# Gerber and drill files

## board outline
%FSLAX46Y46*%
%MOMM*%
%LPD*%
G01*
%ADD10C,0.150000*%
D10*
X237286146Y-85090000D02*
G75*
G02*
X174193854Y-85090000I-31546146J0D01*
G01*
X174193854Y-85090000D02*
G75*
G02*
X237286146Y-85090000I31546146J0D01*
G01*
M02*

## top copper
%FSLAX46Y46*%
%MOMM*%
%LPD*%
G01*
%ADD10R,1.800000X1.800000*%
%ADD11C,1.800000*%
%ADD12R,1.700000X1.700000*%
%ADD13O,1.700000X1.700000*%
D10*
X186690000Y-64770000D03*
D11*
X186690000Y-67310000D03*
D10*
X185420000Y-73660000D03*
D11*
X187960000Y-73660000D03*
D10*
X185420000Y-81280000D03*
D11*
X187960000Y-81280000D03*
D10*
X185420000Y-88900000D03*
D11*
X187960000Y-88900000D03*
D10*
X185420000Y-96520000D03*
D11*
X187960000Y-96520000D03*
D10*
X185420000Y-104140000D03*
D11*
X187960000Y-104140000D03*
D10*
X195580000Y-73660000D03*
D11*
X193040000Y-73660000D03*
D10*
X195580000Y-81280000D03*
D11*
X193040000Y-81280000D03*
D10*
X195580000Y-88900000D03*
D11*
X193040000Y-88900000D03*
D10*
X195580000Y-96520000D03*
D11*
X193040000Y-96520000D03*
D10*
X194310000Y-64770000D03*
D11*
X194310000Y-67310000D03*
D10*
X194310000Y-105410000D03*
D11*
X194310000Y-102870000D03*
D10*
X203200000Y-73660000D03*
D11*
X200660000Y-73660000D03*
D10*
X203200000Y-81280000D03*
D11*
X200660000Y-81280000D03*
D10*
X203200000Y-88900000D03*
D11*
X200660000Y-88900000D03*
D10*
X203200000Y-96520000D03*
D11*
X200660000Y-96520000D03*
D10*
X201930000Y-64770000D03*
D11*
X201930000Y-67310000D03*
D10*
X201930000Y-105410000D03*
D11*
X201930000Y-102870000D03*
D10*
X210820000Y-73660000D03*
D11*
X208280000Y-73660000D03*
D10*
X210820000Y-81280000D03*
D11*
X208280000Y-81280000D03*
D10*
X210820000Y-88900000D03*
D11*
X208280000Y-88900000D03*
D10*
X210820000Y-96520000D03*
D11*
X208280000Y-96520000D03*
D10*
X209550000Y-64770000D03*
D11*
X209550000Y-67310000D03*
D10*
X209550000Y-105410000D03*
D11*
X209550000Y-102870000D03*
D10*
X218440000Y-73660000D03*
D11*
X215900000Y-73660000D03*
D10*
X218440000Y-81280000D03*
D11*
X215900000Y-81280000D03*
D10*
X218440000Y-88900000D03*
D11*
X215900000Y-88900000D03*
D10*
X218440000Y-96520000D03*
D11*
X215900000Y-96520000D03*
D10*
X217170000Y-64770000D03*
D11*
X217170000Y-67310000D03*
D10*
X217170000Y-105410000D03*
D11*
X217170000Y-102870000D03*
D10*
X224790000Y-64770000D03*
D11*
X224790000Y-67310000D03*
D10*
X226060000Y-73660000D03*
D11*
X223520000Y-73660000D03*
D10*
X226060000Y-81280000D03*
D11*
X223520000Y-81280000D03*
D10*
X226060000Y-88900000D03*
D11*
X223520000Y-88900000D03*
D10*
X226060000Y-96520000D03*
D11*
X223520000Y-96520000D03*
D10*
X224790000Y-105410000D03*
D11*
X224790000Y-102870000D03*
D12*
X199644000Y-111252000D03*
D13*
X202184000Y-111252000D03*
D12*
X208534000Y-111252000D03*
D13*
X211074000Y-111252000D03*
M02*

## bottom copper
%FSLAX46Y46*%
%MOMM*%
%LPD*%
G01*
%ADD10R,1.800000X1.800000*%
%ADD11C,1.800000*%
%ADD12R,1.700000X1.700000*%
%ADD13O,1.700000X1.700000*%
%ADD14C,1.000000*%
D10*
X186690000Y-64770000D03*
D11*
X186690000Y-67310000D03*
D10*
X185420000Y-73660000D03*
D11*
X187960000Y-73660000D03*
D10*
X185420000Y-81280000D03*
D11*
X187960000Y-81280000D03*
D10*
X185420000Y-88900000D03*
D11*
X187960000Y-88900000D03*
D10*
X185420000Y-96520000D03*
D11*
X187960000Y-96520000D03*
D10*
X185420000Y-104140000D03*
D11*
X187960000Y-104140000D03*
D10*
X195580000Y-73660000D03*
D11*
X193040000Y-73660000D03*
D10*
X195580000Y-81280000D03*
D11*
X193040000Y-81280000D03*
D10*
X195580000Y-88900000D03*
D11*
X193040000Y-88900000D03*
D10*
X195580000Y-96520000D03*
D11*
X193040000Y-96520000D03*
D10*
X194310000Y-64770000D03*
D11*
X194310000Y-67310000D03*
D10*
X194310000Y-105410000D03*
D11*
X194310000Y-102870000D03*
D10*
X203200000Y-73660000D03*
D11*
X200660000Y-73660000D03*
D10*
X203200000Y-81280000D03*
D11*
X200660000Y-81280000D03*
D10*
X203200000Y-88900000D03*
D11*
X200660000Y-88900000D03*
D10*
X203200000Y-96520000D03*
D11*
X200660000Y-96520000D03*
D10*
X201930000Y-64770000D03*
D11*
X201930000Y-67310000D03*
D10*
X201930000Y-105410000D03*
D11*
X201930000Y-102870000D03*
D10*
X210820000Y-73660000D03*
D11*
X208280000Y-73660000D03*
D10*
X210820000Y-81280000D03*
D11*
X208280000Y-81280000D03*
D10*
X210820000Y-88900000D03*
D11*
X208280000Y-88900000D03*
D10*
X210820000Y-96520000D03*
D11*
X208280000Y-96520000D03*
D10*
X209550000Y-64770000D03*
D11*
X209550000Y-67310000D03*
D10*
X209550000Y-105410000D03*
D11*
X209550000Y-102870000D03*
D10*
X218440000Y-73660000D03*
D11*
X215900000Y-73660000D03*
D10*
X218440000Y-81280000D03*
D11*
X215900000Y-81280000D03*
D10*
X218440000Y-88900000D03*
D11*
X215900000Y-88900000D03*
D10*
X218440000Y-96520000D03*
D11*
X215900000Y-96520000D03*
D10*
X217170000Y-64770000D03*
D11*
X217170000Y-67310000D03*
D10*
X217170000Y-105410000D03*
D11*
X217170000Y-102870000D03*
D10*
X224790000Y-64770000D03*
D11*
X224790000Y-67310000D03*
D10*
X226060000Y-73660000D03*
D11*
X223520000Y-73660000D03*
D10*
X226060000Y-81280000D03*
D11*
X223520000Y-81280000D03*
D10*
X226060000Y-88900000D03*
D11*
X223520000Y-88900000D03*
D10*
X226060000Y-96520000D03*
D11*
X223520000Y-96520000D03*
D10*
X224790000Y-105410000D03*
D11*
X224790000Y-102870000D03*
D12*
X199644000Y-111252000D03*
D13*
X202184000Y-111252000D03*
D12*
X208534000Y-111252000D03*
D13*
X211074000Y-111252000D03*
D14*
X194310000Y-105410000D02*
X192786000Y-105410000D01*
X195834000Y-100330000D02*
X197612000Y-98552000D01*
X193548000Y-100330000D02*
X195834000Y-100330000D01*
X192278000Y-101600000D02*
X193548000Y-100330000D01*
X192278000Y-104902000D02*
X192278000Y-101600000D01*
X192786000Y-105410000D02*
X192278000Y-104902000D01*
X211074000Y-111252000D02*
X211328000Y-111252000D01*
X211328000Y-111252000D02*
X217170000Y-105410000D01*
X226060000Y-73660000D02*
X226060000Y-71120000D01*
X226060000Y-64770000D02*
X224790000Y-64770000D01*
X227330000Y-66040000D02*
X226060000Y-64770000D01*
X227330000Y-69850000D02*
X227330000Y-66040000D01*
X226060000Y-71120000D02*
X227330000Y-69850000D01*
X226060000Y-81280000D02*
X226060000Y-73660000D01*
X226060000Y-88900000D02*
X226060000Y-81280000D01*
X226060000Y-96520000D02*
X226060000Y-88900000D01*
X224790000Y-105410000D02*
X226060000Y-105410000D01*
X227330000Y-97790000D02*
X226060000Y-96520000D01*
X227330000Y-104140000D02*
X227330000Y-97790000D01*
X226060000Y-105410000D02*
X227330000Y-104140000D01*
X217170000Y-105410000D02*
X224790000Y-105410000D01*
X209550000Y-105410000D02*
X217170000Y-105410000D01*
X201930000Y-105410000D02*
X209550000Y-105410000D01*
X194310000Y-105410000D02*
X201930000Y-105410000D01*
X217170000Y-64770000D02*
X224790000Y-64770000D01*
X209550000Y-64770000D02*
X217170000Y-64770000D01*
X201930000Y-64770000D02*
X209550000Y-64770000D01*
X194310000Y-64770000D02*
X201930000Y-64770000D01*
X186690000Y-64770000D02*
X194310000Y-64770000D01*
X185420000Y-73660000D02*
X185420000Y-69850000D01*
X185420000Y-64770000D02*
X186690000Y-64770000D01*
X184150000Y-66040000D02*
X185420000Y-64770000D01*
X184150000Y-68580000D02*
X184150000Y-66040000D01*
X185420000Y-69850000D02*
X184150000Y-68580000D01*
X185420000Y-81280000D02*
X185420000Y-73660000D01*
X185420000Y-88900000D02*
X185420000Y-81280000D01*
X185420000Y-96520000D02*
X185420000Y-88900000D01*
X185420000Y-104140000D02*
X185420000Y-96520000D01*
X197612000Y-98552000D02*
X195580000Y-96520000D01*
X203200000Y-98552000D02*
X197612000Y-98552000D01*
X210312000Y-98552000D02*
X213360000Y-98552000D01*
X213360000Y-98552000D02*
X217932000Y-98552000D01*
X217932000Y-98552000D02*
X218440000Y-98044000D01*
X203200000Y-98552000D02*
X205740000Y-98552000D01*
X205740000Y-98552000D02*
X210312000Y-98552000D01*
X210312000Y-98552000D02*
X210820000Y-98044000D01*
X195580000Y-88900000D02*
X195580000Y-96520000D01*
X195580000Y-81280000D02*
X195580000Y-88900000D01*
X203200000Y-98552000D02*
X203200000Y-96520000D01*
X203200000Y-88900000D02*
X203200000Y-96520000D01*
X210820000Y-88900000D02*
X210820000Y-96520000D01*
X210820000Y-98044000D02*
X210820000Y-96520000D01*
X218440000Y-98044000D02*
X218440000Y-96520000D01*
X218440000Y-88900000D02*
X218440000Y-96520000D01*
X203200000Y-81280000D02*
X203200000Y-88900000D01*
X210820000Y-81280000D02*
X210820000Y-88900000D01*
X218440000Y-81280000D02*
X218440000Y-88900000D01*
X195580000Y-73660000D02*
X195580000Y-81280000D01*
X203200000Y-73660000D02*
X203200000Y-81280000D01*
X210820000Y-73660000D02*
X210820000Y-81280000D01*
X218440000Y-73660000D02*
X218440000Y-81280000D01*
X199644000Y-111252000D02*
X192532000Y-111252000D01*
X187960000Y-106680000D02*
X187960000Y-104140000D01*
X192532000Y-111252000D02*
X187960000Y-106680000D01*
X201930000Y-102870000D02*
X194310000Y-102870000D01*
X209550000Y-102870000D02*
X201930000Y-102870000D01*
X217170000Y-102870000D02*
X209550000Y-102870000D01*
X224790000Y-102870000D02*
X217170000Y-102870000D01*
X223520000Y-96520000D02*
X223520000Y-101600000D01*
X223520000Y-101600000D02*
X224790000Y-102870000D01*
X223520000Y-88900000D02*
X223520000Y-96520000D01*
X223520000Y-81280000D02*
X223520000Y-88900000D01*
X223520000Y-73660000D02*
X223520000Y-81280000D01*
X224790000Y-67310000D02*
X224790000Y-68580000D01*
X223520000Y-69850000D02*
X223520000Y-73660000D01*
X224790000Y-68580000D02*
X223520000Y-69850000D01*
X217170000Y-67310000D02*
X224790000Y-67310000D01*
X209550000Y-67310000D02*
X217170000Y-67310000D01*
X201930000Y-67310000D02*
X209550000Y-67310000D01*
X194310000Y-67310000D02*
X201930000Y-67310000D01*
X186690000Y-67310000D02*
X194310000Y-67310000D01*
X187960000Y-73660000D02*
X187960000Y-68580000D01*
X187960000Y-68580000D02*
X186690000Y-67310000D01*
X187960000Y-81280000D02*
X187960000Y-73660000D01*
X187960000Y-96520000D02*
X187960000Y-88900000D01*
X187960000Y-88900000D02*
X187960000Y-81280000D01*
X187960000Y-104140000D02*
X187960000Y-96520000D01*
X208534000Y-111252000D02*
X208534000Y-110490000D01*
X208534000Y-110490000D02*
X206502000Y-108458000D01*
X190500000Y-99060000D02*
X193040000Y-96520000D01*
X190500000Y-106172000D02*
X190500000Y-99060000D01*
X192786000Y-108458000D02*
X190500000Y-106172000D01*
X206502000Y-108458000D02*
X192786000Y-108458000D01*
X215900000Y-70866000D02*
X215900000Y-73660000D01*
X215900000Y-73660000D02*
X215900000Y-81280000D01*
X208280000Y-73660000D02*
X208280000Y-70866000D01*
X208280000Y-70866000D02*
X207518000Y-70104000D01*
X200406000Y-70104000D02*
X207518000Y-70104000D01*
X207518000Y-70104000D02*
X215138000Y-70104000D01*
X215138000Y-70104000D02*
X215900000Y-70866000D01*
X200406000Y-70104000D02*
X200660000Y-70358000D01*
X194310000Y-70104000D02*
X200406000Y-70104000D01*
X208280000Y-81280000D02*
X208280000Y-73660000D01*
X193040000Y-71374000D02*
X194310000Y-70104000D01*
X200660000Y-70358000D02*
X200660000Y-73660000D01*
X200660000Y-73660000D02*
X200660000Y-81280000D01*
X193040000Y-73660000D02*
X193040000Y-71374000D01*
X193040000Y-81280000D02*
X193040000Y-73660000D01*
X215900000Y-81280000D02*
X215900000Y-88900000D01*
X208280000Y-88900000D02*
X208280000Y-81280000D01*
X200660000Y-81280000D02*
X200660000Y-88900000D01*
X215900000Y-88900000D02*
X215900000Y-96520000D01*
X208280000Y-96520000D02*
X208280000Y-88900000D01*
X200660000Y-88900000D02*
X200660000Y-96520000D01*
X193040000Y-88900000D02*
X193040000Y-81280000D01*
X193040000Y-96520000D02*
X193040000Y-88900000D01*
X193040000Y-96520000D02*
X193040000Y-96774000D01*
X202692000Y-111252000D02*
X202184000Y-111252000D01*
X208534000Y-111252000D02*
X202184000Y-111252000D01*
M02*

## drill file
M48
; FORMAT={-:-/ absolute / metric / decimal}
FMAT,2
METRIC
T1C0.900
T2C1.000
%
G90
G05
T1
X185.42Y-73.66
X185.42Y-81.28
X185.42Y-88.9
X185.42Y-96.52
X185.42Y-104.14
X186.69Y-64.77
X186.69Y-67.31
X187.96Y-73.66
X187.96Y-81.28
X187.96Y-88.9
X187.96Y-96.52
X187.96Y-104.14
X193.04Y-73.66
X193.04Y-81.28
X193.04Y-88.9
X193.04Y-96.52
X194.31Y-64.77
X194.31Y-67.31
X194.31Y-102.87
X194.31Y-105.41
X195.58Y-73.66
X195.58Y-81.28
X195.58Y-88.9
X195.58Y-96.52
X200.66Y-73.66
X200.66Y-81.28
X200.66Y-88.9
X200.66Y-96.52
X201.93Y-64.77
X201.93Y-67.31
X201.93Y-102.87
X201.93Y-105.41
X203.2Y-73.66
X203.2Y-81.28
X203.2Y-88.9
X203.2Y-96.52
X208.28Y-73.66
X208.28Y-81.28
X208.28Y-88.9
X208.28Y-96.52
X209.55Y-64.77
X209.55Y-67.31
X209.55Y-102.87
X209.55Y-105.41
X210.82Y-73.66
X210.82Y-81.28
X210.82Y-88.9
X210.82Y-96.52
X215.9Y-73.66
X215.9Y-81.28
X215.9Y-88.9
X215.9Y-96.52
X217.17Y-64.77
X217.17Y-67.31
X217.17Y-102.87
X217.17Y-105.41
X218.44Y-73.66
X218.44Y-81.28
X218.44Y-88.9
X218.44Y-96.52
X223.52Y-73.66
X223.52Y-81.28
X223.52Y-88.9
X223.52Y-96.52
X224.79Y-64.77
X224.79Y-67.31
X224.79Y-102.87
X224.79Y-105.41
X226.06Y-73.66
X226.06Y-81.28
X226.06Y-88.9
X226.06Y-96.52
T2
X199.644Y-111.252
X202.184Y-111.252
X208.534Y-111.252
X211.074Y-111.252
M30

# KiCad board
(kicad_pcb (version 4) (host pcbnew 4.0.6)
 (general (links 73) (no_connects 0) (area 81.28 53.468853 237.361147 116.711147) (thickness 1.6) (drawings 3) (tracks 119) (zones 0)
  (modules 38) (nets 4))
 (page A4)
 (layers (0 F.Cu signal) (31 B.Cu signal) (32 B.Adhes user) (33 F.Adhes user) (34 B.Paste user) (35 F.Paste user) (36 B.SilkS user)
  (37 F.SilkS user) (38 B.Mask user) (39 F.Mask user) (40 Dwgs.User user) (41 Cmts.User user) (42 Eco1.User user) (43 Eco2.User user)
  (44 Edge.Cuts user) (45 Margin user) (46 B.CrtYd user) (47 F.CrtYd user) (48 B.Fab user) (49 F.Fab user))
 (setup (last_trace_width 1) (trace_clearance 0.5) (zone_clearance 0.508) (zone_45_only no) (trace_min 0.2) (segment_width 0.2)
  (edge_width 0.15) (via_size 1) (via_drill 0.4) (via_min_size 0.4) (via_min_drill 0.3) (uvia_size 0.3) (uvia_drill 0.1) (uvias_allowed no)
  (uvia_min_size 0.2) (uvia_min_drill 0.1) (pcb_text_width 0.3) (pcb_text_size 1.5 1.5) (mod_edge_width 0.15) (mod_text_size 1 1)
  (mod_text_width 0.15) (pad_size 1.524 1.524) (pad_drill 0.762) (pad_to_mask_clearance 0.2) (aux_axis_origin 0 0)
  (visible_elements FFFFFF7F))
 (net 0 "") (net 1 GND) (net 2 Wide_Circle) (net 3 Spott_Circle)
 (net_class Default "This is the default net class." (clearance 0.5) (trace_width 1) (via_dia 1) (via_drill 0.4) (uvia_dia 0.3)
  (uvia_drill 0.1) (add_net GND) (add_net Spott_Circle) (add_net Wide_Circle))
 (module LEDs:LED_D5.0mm (layer F.Cu) (at 186.69 64.77 270)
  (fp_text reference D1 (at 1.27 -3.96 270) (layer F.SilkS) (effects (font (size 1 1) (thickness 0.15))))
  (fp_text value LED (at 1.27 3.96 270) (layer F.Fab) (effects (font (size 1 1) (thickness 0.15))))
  (pad 1 thru_hole rect (at 0 0 270) (size 1.8 1.8) (drill 0.9) (layers *.Cu *.Mask) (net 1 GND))
  (pad 2 thru_hole circle (at 2.54 0 270) (size 1.8 1.8) (drill 0.9) (layers *.Cu *.Mask) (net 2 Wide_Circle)))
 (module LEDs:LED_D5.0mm (layer F.Cu) (at 185.42 73.66)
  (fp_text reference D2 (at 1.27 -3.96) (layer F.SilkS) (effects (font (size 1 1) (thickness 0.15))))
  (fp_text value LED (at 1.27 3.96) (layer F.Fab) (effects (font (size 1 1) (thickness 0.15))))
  (pad 1 thru_hole rect (at 0 0) (size 1.8 1.8) (drill 0.9) (layers *.Cu *.Mask) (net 1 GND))
  (pad 2 thru_hole circle (at 2.54 0) (size 1.8 1.8) (drill 0.9) (layers *.Cu *.Mask) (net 2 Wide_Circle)))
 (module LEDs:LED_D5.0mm (layer F.Cu) (at 185.42 81.28)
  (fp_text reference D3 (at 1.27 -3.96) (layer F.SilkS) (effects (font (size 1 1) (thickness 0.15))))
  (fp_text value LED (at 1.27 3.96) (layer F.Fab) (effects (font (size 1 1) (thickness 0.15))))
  (pad 1 thru_hole rect (at 0 0) (size 1.8 1.8) (drill 0.9) (layers *.Cu *.Mask) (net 1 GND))
  (pad 2 thru_hole circle (at 2.54 0) (size 1.8 1.8) (drill 0.9) (layers *.Cu *.Mask) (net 2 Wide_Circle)))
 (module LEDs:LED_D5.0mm (layer F.Cu) (at 185.42 88.9)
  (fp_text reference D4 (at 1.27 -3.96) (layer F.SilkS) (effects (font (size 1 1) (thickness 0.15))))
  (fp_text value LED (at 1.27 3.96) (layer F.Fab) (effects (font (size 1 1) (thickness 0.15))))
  (pad 1 thru_hole rect (at 0 0) (size 1.8 1.8) (drill 0.9) (layers *.Cu *.Mask) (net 1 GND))
  (pad 2 thru_hole circle (at 2.54 0) (size 1.8 1.8) (drill 0.9) (layers *.Cu *.Mask) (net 2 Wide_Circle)))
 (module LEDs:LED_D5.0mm (layer F.Cu) (at 185.42 96.52)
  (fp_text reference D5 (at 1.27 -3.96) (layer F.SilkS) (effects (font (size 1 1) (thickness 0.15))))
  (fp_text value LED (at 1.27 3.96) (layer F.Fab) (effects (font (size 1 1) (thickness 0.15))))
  (pad 1 thru_hole rect (at 0 0) (size 1.8 1.8) (drill 0.9) (layers *.Cu *.Mask) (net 1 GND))
  (pad 2 thru_hole circle (at 2.54 0) (size 1.8 1.8) (drill 0.9) (layers *.Cu *.Mask) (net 2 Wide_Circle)))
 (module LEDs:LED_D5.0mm (layer F.Cu) (at 185.42 104.14)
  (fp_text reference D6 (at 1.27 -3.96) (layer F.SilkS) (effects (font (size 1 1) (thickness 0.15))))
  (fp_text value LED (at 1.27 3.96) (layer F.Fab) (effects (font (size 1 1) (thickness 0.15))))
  (pad 1 thru_hole rect (at 0 0) (size 1.8 1.8) (drill 0.9) (layers *.Cu *.Mask) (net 1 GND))
  (pad 2 thru_hole circle (at 2.54 0) (size 1.8 1.8) (drill 0.9) (layers *.Cu *.Mask) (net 2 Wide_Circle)))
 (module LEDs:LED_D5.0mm (layer F.Cu) (at 195.58 73.66 180)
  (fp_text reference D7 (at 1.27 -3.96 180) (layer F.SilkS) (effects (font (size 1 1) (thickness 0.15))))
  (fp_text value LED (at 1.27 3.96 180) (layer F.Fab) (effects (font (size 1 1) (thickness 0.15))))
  (pad 1 thru_hole rect (at 0 0 180) (size 1.8 1.8) (drill 0.9) (layers *.Cu *.Mask) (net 1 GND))
  (pad 2 thru_hole circle (at 2.54 0 180) (size 1.8 1.8) (drill 0.9) (layers *.Cu *.Mask) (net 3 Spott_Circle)))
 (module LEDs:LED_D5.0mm (layer F.Cu) (at 195.58 81.28 180)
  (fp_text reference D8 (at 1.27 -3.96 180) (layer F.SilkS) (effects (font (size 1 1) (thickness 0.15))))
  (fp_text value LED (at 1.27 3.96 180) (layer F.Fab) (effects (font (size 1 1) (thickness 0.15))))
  (pad 1 thru_hole rect (at 0 0 180) (size 1.8 1.8) (drill 0.9) (layers *.Cu *.Mask) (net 1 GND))
  (pad 2 thru_hole circle (at 2.54 0 180) (size 1.8 1.8) (drill 0.9) (layers *.Cu *.Mask) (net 3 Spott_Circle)))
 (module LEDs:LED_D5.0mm (layer F.Cu) (at 195.58 88.9 180)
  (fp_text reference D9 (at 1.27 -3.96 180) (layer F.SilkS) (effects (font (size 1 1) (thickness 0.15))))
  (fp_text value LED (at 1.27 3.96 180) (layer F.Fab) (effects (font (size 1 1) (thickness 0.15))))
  (pad 1 thru_hole rect (at 0 0 180) (size 1.8 1.8) (drill 0.9) (layers *.Cu *.Mask) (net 1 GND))
  (pad 2 thru_hole circle (at 2.54 0 180) (size 1.8 1.8) (drill 0.9) (layers *.Cu *.Mask) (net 3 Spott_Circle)))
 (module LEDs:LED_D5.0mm (layer F.Cu) (at 195.58 96.52 180)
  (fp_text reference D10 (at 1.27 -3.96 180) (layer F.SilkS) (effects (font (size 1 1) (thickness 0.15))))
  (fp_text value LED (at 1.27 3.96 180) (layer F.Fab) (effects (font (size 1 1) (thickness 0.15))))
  (pad 1 thru_hole rect (at 0 0 180) (size 1.8 1.8) (drill 0.9) (layers *.Cu *.Mask) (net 1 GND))
  (pad 2 thru_hole circle (at 2.54 0 180) (size 1.8 1.8) (drill 0.9) (layers *.Cu *.Mask) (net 3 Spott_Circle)))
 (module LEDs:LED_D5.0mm (layer F.Cu) (at 194.31 64.77 270)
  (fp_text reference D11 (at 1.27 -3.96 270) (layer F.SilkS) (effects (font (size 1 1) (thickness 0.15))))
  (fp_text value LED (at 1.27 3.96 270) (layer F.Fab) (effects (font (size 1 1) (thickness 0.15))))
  (pad 1 thru_hole rect (at 0 0 270) (size 1.8 1.8) (drill 0.9) (layers *.Cu *.Mask) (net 1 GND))
  (pad 2 thru_hole circle (at 2.54 0 270) (size 1.8 1.8) (drill 0.9) (layers *.Cu *.Mask) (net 2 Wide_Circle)))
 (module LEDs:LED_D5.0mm (layer F.Cu) (at 194.31 105.41 90)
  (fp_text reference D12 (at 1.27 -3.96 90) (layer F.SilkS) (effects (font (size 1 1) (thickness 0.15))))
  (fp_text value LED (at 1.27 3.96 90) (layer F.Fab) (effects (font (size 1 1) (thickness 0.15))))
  (pad 1 thru_hole rect (at 0 0 90) (size 1.8 1.8) (drill 0.9) (layers *.Cu *.Mask) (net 1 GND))
  (pad 2 thru_hole circle (at 2.54 0 90) (size 1.8 1.8) (drill 0.9) (layers *.Cu *.Mask) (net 2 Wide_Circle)))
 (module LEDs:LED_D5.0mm (layer F.Cu) (at 203.2 73.66 180)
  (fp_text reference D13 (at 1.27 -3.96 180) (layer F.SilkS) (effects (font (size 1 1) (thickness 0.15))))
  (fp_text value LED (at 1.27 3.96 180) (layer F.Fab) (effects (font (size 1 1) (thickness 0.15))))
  (pad 1 thru_hole rect (at 0 0 180) (size 1.8 1.8) (drill 0.9) (layers *.Cu *.Mask) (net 1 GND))
  (pad 2 thru_hole circle (at 2.54 0 180) (size 1.8 1.8) (drill 0.9) (layers *.Cu *.Mask) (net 3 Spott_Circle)))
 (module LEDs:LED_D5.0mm (layer F.Cu) (at 203.2 81.28 180)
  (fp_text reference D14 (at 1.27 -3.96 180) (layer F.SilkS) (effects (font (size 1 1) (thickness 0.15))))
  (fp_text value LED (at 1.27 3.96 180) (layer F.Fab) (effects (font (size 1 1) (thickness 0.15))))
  (pad 1 thru_hole rect (at 0 0 180) (size 1.8 1.8) (drill 0.9) (layers *.Cu *.Mask) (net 1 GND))
  (pad 2 thru_hole circle (at 2.54 0 180) (size 1.8 1.8) (drill 0.9) (layers *.Cu *.Mask) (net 3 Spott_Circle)))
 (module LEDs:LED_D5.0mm (layer F.Cu) (at 203.2 88.9 180)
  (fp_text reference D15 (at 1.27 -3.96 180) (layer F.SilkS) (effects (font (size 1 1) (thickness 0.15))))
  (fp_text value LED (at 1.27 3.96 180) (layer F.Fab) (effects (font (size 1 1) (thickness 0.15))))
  (pad 1 thru_hole rect (at 0 0 180) (size 1.8 1.8) (drill 0.9) (layers *.Cu *.Mask) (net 1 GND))
  (pad 2 thru_hole circle (at 2.54 0 180) (size 1.8 1.8) (drill 0.9) (layers *.Cu *.Mask) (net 3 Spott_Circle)))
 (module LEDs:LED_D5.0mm (layer F.Cu) (at 203.2 96.52 180)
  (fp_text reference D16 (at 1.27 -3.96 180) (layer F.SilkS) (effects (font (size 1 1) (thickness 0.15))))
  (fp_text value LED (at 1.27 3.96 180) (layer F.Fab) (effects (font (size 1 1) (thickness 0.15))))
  (pad 1 thru_hole rect (at 0 0 180) (size 1.8 1.8) (drill 0.9) (layers *.Cu *.Mask) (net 1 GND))
  (pad 2 thru_hole circle (at 2.54 0 180) (size 1.8 1.8) (drill 0.9) (layers *.Cu *.Mask) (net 3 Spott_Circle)))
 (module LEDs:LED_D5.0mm (layer F.Cu) (at 201.93 64.77 270)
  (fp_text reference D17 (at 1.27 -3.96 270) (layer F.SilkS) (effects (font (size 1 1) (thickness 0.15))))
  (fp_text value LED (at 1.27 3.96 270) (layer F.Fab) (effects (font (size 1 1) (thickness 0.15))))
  (pad 1 thru_hole rect (at 0 0 270) (size 1.8 1.8) (drill 0.9) (layers *.Cu *.Mask) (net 1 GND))
  (pad 2 thru_hole circle (at 2.54 0 270) (size 1.8 1.8) (drill 0.9) (layers *.Cu *.Mask) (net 2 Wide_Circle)))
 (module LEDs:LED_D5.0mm (layer F.Cu) (at 201.93 105.41 90)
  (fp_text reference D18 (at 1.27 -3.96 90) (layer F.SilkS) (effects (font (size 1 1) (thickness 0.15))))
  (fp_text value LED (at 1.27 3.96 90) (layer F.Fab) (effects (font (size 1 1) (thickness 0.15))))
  (pad 1 thru_hole rect (at 0 0 90) (size 1.8 1.8) (drill 0.9) (layers *.Cu *.Mask) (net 1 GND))
  (pad 2 thru_hole circle (at 2.54 0 90) (size 1.8 1.8) (drill 0.9) (layers *.Cu *.Mask) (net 2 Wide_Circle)))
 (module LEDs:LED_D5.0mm (layer F.Cu) (at 210.82 73.66 180)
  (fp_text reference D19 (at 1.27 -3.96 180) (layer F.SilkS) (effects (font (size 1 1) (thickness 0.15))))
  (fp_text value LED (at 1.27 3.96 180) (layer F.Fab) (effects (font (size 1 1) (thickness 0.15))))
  (pad 1 thru_hole rect (at 0 0 180) (size 1.8 1.8) (drill 0.9) (layers *.Cu *.Mask) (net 1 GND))
  (pad 2 thru_hole circle (at 2.54 0 180) (size 1.8 1.8) (drill 0.9) (layers *.Cu *.Mask) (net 3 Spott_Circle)))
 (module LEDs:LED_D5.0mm (layer F.Cu) (at 210.82 81.28 180)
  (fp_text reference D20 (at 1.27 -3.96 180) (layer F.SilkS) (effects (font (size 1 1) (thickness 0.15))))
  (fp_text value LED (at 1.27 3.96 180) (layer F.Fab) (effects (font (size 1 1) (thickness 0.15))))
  (pad 1 thru_hole rect (at 0 0 180) (size 1.8 1.8) (drill 0.9) (layers *.Cu *.Mask) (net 1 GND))
  (pad 2 thru_hole circle (at 2.54 0 180) (size 1.8 1.8) (drill 0.9) (layers *.Cu *.Mask) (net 3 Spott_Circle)))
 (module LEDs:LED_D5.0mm (layer F.Cu) (at 210.82 88.9 180)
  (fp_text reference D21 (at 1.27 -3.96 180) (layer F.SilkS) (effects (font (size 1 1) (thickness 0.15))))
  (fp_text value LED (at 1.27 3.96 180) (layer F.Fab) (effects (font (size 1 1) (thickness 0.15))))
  (pad 1 thru_hole rect (at 0 0 180) (size 1.8 1.8) (drill 0.9) (layers *.Cu *.Mask) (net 1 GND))
  (pad 2 thru_hole circle (at 2.54 0 180) (size 1.8 1.8) (drill 0.9) (layers *.Cu *.Mask) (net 3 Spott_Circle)))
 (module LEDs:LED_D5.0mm (layer F.Cu) (at 210.82 96.52 180)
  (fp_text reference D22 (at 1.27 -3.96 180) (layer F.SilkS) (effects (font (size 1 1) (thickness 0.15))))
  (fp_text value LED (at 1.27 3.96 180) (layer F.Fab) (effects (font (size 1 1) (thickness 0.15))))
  (pad 1 thru_hole rect (at 0 0 180) (size 1.8 1.8) (drill 0.9) (layers *.Cu *.Mask) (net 1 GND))
  (pad 2 thru_hole circle (at 2.54 0 180) (size 1.8 1.8) (drill 0.9) (layers *.Cu *.Mask) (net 3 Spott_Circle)))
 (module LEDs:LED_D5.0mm (layer F.Cu) (at 209.55 64.77 270)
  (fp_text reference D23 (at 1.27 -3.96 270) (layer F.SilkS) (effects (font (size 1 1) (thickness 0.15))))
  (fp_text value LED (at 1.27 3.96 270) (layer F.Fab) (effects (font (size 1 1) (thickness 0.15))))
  (pad 1 thru_hole rect (at 0 0 270) (size 1.8 1.8) (drill 0.9) (layers *.Cu *.Mask) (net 1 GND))
  (pad 2 thru_hole circle (at 2.54 0 270) (size 1.8 1.8) (drill 0.9) (layers *.Cu *.Mask) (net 2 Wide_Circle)))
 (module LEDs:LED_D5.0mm (layer F.Cu) (at 209.55 105.41 90)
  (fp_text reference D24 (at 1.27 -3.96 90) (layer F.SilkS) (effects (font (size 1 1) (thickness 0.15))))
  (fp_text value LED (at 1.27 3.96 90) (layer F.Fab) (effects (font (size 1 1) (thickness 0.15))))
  (pad 1 thru_hole rect (at 0 0 90) (size 1.8 1.8) (drill 0.9) (layers *.Cu *.Mask) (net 1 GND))
  (pad 2 thru_hole circle (at 2.54 0 90) (size 1.8 1.8) (drill 0.9) (layers *.Cu *.Mask) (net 2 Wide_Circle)))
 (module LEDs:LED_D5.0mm (layer F.Cu) (at 218.44 73.66 180)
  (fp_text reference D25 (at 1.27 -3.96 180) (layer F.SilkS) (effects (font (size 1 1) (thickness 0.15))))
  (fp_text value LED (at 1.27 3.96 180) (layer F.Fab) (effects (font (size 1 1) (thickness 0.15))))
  (pad 1 thru_hole rect (at 0 0 180) (size 1.8 1.8) (drill 0.9) (layers *.Cu *.Mask) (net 1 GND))
  (pad 2 thru_hole circle (at 2.54 0 180) (size 1.8 1.8) (drill 0.9) (layers *.Cu *.Mask) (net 3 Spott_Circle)))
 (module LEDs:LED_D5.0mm (layer F.Cu) (at 218.44 81.28 180)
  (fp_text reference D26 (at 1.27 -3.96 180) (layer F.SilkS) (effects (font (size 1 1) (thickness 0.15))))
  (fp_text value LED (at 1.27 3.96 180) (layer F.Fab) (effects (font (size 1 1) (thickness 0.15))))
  (pad 1 thru_hole rect (at 0 0 180) (size 1.8 1.8) (drill 0.9) (layers *.Cu *.Mask) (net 1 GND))
  (pad 2 thru_hole circle (at 2.54 0 180) (size 1.8 1.8) (drill 0.9) (layers *.Cu *.Mask) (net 3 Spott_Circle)))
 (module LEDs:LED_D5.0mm (layer F.Cu) (at 218.44 88.9 180)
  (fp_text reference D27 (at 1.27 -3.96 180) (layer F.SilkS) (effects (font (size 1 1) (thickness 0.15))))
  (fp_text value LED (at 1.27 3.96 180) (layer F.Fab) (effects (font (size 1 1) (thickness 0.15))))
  (pad 1 thru_hole rect (at 0 0 180) (size 1.8 1.8) (drill 0.9) (layers *.Cu *.Mask) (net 1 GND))
  (pad 2 thru_hole circle (at 2.54 0 180) (size 1.8 1.8) (drill 0.9) (layers *.Cu *.Mask) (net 3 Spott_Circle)))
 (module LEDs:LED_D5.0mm (layer F.Cu) (at 218.44 96.52 180)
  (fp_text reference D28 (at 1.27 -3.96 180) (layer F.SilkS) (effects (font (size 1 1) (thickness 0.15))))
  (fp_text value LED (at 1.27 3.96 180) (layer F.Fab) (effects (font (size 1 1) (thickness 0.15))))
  (pad 1 thru_hole rect (at 0 0 180) (size 1.8 1.8) (drill 0.9) (layers *.Cu *.Mask) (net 1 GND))
  (pad 2 thru_hole circle (at 2.54 0 180) (size 1.8 1.8) (drill 0.9) (layers *.Cu *.Mask) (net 3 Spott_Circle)))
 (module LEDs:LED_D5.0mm (layer F.Cu) (at 217.17 64.77 270)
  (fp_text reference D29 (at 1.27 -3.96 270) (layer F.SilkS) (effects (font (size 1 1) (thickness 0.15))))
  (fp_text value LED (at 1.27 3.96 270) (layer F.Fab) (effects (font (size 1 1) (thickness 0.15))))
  (pad 1 thru_hole rect (at 0 0 270) (size 1.8 1.8) (drill 0.9) (layers *.Cu *.Mask) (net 1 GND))
  (pad 2 thru_hole circle (at 2.54 0 270) (size 1.8 1.8) (drill 0.9) (layers *.Cu *.Mask) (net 2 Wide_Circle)))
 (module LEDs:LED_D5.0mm (layer F.Cu) (at 217.17 105.41 90)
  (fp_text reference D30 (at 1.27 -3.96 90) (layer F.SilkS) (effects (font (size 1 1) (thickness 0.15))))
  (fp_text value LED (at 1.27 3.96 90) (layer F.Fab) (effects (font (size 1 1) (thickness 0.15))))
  (pad 1 thru_hole rect (at 0 0 90) (size 1.8 1.8) (drill 0.9) (layers *.Cu *.Mask) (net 1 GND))
  (pad 2 thru_hole circle (at 2.54 0 90) (size 1.8 1.8) (drill 0.9) (layers *.Cu *.Mask) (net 2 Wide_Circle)))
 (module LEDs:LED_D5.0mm (layer F.Cu) (at 224.79 64.77 270)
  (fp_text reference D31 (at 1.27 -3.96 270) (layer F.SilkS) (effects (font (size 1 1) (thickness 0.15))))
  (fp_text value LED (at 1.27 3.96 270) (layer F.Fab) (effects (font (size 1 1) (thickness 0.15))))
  (pad 1 thru_hole rect (at 0 0 270) (size 1.8 1.8) (drill 0.9) (layers *.Cu *.Mask) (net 1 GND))
  (pad 2 thru_hole circle (at 2.54 0 270) (size 1.8 1.8) (drill 0.9) (layers *.Cu *.Mask) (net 2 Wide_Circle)))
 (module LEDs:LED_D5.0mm (layer F.Cu) (at 226.06 73.66 180)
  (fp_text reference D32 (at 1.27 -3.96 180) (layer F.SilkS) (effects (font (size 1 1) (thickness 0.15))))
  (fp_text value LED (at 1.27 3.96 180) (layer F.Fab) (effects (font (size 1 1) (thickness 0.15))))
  (pad 1 thru_hole rect (at 0 0 180) (size 1.8 1.8) (drill 0.9) (layers *.Cu *.Mask) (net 1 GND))
  (pad 2 thru_hole circle (at 2.54 0 180) (size 1.8 1.8) (drill 0.9) (layers *.Cu *.Mask) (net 2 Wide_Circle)))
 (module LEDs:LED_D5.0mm (layer F.Cu) (at 226.06 81.28 180)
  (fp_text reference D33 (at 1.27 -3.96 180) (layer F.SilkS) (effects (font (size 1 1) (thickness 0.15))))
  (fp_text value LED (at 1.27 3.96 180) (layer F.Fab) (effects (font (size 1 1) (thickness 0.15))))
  (pad 1 thru_hole rect (at 0 0 180) (size 1.8 1.8) (drill 0.9) (layers *.Cu *.Mask) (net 1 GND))
  (pad 2 thru_hole circle (at 2.54 0 180) (size 1.8 1.8) (drill 0.9) (layers *.Cu *.Mask) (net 2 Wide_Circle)))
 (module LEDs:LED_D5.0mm (layer F.Cu) (at 226.06 88.9 180)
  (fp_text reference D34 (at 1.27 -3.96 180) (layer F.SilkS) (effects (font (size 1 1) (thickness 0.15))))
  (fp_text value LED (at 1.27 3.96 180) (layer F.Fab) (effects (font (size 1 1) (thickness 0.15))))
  (pad 1 thru_hole rect (at 0 0 180) (size 1.8 1.8) (drill 0.9) (layers *.Cu *.Mask) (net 1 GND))
  (pad 2 thru_hole circle (at 2.54 0 180) (size 1.8 1.8) (drill 0.9) (layers *.Cu *.Mask) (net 2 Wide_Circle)))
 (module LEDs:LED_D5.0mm (layer F.Cu) (at 226.06 96.52 180)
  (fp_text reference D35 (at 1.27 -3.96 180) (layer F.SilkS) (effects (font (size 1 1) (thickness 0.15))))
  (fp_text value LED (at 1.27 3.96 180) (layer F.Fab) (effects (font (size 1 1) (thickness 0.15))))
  (pad 1 thru_hole rect (at 0 0 180) (size 1.8 1.8) (drill 0.9) (layers *.Cu *.Mask) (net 1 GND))
  (pad 2 thru_hole circle (at 2.54 0 180) (size 1.8 1.8) (drill 0.9) (layers *.Cu *.Mask) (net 2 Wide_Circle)))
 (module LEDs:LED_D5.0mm (layer F.Cu) (at 224.79 105.41 90)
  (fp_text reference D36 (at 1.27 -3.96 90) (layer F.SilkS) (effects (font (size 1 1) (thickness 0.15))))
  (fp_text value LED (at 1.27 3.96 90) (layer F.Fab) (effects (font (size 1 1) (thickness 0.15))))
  (pad 1 thru_hole rect (at 0 0 90) (size 1.8 1.8) (drill 0.9) (layers *.Cu *.Mask) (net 1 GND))
  (pad 2 thru_hole circle (at 2.54 0 90) (size 1.8 1.8) (drill 0.9) (layers *.Cu *.Mask) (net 2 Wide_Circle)))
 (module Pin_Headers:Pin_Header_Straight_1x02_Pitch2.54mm (layer F.Cu) (at 199.644 111.252 90)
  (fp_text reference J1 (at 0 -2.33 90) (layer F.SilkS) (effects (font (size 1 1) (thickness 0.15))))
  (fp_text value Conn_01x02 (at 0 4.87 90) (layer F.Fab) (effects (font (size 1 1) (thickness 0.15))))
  (pad 1 thru_hole rect (at 0 0 90) (size 1.7 1.7) (drill 1) (layers *.Cu *.Mask) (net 2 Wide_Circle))
  (pad 2 thru_hole oval (at 0 2.54 90) (size 1.7 1.7) (drill 1) (layers *.Cu *.Mask) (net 3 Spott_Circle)))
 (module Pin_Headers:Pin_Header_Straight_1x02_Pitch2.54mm (layer F.Cu) (at 208.534 111.252 90)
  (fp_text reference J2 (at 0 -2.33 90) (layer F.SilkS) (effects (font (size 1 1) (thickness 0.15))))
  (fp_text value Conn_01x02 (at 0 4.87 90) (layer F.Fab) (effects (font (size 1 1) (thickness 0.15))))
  (pad 1 thru_hole rect (at 0 0 90) (size 1.7 1.7) (drill 1) (layers *.Cu *.Mask) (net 3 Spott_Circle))
  (pad 2 thru_hole oval (at 0 2.54 90) (size 1.7 1.7) (drill 1) (layers *.Cu *.Mask) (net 1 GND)))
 (gr_circle (center 205.74 85.09) (end 229.87 105.41) (layer Edge.Cuts) (width 0.15))
 (segment (start 194.31 105.41) (end 192.786 105.41) (width 1) (layer B.Cu) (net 1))
 (segment (start 195.834 100.33) (end 197.612 98.552) (width 1) (layer B.Cu) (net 1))
 (segment (start 193.548 100.33) (end 195.834 100.33) (width 1) (layer B.Cu) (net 1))
 (segment (start 192.278 101.6) (end 193.548 100.33) (width 1) (layer B.Cu) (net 1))
 (segment (start 192.278 104.902) (end 192.278 101.6) (width 1) (layer B.Cu) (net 1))
 (segment (start 192.786 105.41) (end 192.278 104.902) (width 1) (layer B.Cu) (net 1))
 (segment (start 211.074 111.252) (end 211.328 111.252) (width 1) (layer B.Cu) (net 1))
 (segment (start 211.328 111.252) (end 217.17 105.41) (width 1) (layer B.Cu) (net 1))
 (segment (start 226.06 73.66) (end 226.06 71.12) (width 1) (layer B.Cu) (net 1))
 (segment (start 226.06 64.77) (end 224.79 64.77) (width 1) (layer B.Cu) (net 1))
 (segment (start 227.33 66.04) (end 226.06 64.77) (width 1) (layer B.Cu) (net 1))
 (segment (start 227.33 69.85) (end 227.33 66.04) (width 1) (layer B.Cu) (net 1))
 (segment (start 226.06 71.12) (end 227.33 69.85) (width 1) (layer B.Cu) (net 1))
 (segment (start 226.06 81.28) (end 226.06 73.66) (width 1) (layer B.Cu) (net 1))
 (segment (start 226.06 88.9) (end 226.06 81.28) (width 1) (layer B.Cu) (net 1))
 (segment (start 226.06 96.52) (end 226.06 88.9) (width 1) (layer B.Cu) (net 1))
 (segment (start 224.79 105.41) (end 226.06 105.41) (width 1) (layer B.Cu) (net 1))
 (segment (start 227.33 97.79) (end 226.06 96.52) (width 1) (layer B.Cu) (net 1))
 (segment (start 227.33 104.14) (end 227.33 97.79) (width 1) (layer B.Cu) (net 1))
 (segment (start 226.06 105.41) (end 227.33 104.14) (width 1) (layer B.Cu) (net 1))
 (segment (start 217.17 105.41) (end 224.79 105.41) (width 1) (layer B.Cu) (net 1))
 (segment (start 209.55 105.41) (end 217.17 105.41) (width 1) (layer B.Cu) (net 1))
 (segment (start 201.93 105.41) (end 209.55 105.41) (width 1) (layer B.Cu) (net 1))
 (segment (start 194.31 105.41) (end 201.93 105.41) (width 1) (layer B.Cu) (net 1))
 (segment (start 217.17 64.77) (end 224.79 64.77) (width 1) (layer B.Cu) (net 1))
 (segment (start 209.55 64.77) (end 217.17 64.77) (width 1) (layer B.Cu) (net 1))
 (segment (start 201.93 64.77) (end 209.55 64.77) (width 1) (layer B.Cu) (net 1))
 (segment (start 194.31 64.77) (end 201.93 64.77) (width 1) (layer B.Cu) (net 1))
 (segment (start 186.69 64.77) (end 194.31 64.77) (width 1) (layer B.Cu) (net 1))
 (segment (start 185.42 73.66) (end 185.42 69.85) (width 1) (layer B.Cu) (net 1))
 (segment (start 185.42 64.77) (end 186.69 64.77) (width 1) (layer B.Cu) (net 1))
 (segment (start 184.15 66.04) (end 185.42 64.77) (width 1) (layer B.Cu) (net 1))
 (segment (start 184.15 68.58) (end 184.15 66.04) (width 1) (layer B.Cu) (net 1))
 (segment (start 185.42 69.85) (end 184.15 68.58) (width 1) (layer B.Cu) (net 1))
 (segment (start 185.42 81.28) (end 185.42 73.66) (width 1) (layer B.Cu) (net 1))
 (segment (start 185.42 88.9) (end 185.42 81.28) (width 1) (layer B.Cu) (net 1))
 (segment (start 185.42 96.52) (end 185.42 88.9) (width 1) (layer B.Cu) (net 1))
 (segment (start 185.42 104.14) (end 185.42 96.52) (width 1) (layer B.Cu) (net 1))
 (segment (start 197.612 98.552) (end 195.58 96.52) (width 1) (layer B.Cu) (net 1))
 (segment (start 203.2 98.552) (end 197.612 98.552) (width 1) (layer B.Cu) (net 1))
 (segment (start 210.312 98.552) (end 213.36 98.552) (width 1) (layer B.Cu) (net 1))
 (segment (start 213.36 98.552) (end 217.932 98.552) (width 1) (layer B.Cu) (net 1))
 (segment (start 217.932 98.552) (end 218.44 98.044) (width 1) (layer B.Cu) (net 1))
 (segment (start 203.2 98.552) (end 205.74 98.552) (width 1) (layer B.Cu) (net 1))
 (segment (start 205.74 98.552) (end 210.312 98.552) (width 1) (layer B.Cu) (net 1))
 (segment (start 210.312 98.552) (end 210.82 98.044) (width 1) (layer B.Cu) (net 1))
 (segment (start 195.58 88.9) (end 195.58 96.52) (width 1) (layer B.Cu) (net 1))
 (segment (start 195.58 81.28) (end 195.58 88.9) (width 1) (layer B.Cu) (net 1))
 (segment (start 203.2 98.552) (end 203.2 96.52) (width 1) (layer B.Cu) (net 1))
 (segment (start 203.2 88.9) (end 203.2 96.52) (width 1) (layer B.Cu) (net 1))
 (segment (start 210.82 88.9) (end 210.82 96.52) (width 1) (layer B.Cu) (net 1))
 (segment (start 210.82 98.044) (end 210.82 96.52) (width 1) (layer B.Cu) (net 1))
 (segment (start 218.44 98.044) (end 218.44 96.52) (width 1) (layer B.Cu) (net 1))
 (segment (start 218.44 88.9) (end 218.44 96.52) (width 1) (layer B.Cu) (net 1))
 (segment (start 203.2 81.28) (end 203.2 88.9) (width 1) (layer B.Cu) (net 1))
 (segment (start 210.82 81.28) (end 210.82 88.9) (width 1) (layer B.Cu) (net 1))
 (segment (start 218.44 81.28) (end 218.44 88.9) (width 1) (layer B.Cu) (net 1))
 (segment (start 195.58 73.66) (end 195.58 81.28) (width 1) (layer B.Cu) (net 1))
 (segment (start 203.2 73.66) (end 203.2 81.28) (width 1) (layer B.Cu) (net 1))
 (segment (start 210.82 73.66) (end 210.82 81.28) (width 1) (layer B.Cu) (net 1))
 (segment (start 218.44 73.66) (end 218.44 81.28) (width 1) (layer B.Cu) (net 1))
 (segment (start 199.644 111.252) (end 192.532 111.252) (width 1) (layer B.Cu) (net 2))
 (segment (start 187.96 106.68) (end 187.96 104.14) (width 1) (layer B.Cu) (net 2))
 (segment (start 192.532 111.252) (end 187.96 106.68) (width 1) (layer B.Cu) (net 2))
 (segment (start 201.93 102.87) (end 194.31 102.87) (width 1) (layer B.Cu) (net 2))
 (segment (start 209.55 102.87) (end 201.93 102.87) (width 1) (layer B.Cu) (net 2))
 (segment (start 217.17 102.87) (end 209.55 102.87) (width 1) (layer B.Cu) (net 2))
 (segment (start 224.79 102.87) (end 217.17 102.87) (width 1) (layer B.Cu) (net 2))
 (segment (start 223.52 96.52) (end 223.52 101.6) (width 1) (layer B.Cu) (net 2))
 (segment (start 223.52 101.6) (end 224.79 102.87) (width 1) (layer B.Cu) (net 2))
 (segment (start 223.52 88.9) (end 223.52 96.52) (width 1) (layer B.Cu) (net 2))
 (segment (start 223.52 81.28) (end 223.52 88.9) (width 1) (layer B.Cu) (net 2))
 (segment (start 223.52 73.66) (end 223.52 81.28) (width 1) (layer B.Cu) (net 2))
 (segment (start 224.79 67.31) (end 224.79 68.58) (width 1) (layer B.Cu) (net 2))
 (segment (start 223.52 69.85) (end 223.52 73.66) (width 1) (layer B.Cu) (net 2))
 (segment (start 224.79 68.58) (end 223.52 69.85) (width 1) (layer B.Cu) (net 2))
 (segment (start 217.17 67.31) (end 224.79 67.31) (width 1) (layer B.Cu) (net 2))
 (segment (start 209.55 67.31) (end 217.17 67.31) (width 1) (layer B.Cu) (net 2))
 (segment (start 201.93 67.31) (end 209.55 67.31) (width 1) (layer B.Cu) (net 2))
 (segment (start 194.31 67.31) (end 201.93 67.31) (width 1) (layer B.Cu) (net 2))
 (segment (start 186.69 67.31) (end 194.31 67.31) (width 1) (layer B.Cu) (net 2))
 (segment (start 187.96 73.66) (end 187.96 68.58) (width 1) (layer B.Cu) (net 2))
 (segment (start 187.96 68.58) (end 186.69 67.31) (width 1) (layer B.Cu) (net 2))
 (segment (start 187.96 81.28) (end 187.96 73.66) (width 1) (layer B.Cu) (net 2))
 (segment (start 187.96 96.52) (end 187.96 88.9) (width 1) (layer B.Cu) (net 2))
 (segment (start 187.96 88.9) (end 187.96 81.28) (width 1) (layer B.Cu) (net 2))
 (segment (start 187.96 104.14) (end 187.96 96.52) (width 1) (layer B.Cu) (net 2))
 (segment (start 208.534 111.252) (end 208.534 110.49) (width 1) (layer B.Cu) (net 3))
 (segment (start 208.534 110.49) (end 206.502 108.458) (width 1) (layer B.Cu) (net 3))
 (segment (start 190.5 99.06) (end 193.04 96.52) (width 1) (layer B.Cu) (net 3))
 (segment (start 190.5 106.172) (end 190.5 99.06) (width 1) (layer B.Cu) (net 3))
 (segment (start 192.786 108.458) (end 190.5 106.172) (width 1) (layer B.Cu) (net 3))
 (segment (start 206.502 108.458) (end 192.786 108.458) (width 1) (layer B.Cu) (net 3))
 (segment (start 215.9 70.866) (end 215.9 73.66) (width 1) (layer B.Cu) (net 3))
 (segment (start 215.9 73.66) (end 215.9 81.28) (width 1) (layer B.Cu) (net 3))
 (segment (start 208.28 73.66) (end 208.28 70.866) (width 1) (layer B.Cu) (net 3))
 (segment (start 208.28 70.866) (end 207.518 70.104) (width 1) (layer B.Cu) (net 3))
 (segment (start 200.406 70.104) (end 207.518 70.104) (width 1) (layer B.Cu) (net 3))
 (segment (start 207.518 70.104) (end 215.138 70.104) (width 1) (layer B.Cu) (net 3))
 (segment (start 215.138 70.104) (end 215.9 70.866) (width 1) (layer B.Cu) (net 3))
 (segment (start 200.406 70.104) (end 200.66 70.358) (width 1) (layer B.Cu) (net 3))
 (segment (start 194.31 70.104) (end 200.406 70.104) (width 1) (layer B.Cu) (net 3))
 (segment (start 208.28 81.28) (end 208.28 73.66) (width 1) (layer B.Cu) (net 3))
 (segment (start 193.04 71.374) (end 194.31 70.104) (width 1) (layer B.Cu) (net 3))
 (segment (start 200.66 70.358) (end 200.66 73.66) (width 1) (layer B.Cu) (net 3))
 (segment (start 200.66 73.66) (end 200.66 81.28) (width 1) (layer B.Cu) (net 3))
 (segment (start 193.04 73.66) (end 193.04 71.374) (width 1) (layer B.Cu) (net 3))
 (segment (start 193.04 81.28) (end 193.04 73.66) (width 1) (layer B.Cu) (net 3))
 (segment (start 215.9 81.28) (end 215.9 88.9) (width 1) (layer B.Cu) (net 3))
 (segment (start 208.28 88.9) (end 208.28 81.28) (width 1) (layer B.Cu) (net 3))
 (segment (start 200.66 81.28) (end 200.66 88.9) (width 1) (layer B.Cu) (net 3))
 (segment (start 215.9 88.9) (end 215.9 96.52) (width 1) (layer B.Cu) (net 3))
 (segment (start 208.28 96.52) (end 208.28 88.9) (width 1) (layer B.Cu) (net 3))
 (segment (start 200.66 88.9) (end 200.66 96.52) (width 1) (layer B.Cu) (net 3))
 (segment (start 193.04 88.9) (end 193.04 81.28) (width 1) (layer B.Cu) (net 3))
 (segment (start 193.04 96.52) (end 193.04 88.9) (width 1) (layer B.Cu) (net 3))
 (segment (start 193.04 96.52) (end 193.04 96.774) (width 1) (layer B.Cu) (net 3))
 (segment (start 202.692 111.252) (end 202.184 111.252) (width 1) (layer B.Cu) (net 3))
 (segment (start 208.534 111.252) (end 202.184 111.252) (width 1) (layer B.Cu) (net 3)))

